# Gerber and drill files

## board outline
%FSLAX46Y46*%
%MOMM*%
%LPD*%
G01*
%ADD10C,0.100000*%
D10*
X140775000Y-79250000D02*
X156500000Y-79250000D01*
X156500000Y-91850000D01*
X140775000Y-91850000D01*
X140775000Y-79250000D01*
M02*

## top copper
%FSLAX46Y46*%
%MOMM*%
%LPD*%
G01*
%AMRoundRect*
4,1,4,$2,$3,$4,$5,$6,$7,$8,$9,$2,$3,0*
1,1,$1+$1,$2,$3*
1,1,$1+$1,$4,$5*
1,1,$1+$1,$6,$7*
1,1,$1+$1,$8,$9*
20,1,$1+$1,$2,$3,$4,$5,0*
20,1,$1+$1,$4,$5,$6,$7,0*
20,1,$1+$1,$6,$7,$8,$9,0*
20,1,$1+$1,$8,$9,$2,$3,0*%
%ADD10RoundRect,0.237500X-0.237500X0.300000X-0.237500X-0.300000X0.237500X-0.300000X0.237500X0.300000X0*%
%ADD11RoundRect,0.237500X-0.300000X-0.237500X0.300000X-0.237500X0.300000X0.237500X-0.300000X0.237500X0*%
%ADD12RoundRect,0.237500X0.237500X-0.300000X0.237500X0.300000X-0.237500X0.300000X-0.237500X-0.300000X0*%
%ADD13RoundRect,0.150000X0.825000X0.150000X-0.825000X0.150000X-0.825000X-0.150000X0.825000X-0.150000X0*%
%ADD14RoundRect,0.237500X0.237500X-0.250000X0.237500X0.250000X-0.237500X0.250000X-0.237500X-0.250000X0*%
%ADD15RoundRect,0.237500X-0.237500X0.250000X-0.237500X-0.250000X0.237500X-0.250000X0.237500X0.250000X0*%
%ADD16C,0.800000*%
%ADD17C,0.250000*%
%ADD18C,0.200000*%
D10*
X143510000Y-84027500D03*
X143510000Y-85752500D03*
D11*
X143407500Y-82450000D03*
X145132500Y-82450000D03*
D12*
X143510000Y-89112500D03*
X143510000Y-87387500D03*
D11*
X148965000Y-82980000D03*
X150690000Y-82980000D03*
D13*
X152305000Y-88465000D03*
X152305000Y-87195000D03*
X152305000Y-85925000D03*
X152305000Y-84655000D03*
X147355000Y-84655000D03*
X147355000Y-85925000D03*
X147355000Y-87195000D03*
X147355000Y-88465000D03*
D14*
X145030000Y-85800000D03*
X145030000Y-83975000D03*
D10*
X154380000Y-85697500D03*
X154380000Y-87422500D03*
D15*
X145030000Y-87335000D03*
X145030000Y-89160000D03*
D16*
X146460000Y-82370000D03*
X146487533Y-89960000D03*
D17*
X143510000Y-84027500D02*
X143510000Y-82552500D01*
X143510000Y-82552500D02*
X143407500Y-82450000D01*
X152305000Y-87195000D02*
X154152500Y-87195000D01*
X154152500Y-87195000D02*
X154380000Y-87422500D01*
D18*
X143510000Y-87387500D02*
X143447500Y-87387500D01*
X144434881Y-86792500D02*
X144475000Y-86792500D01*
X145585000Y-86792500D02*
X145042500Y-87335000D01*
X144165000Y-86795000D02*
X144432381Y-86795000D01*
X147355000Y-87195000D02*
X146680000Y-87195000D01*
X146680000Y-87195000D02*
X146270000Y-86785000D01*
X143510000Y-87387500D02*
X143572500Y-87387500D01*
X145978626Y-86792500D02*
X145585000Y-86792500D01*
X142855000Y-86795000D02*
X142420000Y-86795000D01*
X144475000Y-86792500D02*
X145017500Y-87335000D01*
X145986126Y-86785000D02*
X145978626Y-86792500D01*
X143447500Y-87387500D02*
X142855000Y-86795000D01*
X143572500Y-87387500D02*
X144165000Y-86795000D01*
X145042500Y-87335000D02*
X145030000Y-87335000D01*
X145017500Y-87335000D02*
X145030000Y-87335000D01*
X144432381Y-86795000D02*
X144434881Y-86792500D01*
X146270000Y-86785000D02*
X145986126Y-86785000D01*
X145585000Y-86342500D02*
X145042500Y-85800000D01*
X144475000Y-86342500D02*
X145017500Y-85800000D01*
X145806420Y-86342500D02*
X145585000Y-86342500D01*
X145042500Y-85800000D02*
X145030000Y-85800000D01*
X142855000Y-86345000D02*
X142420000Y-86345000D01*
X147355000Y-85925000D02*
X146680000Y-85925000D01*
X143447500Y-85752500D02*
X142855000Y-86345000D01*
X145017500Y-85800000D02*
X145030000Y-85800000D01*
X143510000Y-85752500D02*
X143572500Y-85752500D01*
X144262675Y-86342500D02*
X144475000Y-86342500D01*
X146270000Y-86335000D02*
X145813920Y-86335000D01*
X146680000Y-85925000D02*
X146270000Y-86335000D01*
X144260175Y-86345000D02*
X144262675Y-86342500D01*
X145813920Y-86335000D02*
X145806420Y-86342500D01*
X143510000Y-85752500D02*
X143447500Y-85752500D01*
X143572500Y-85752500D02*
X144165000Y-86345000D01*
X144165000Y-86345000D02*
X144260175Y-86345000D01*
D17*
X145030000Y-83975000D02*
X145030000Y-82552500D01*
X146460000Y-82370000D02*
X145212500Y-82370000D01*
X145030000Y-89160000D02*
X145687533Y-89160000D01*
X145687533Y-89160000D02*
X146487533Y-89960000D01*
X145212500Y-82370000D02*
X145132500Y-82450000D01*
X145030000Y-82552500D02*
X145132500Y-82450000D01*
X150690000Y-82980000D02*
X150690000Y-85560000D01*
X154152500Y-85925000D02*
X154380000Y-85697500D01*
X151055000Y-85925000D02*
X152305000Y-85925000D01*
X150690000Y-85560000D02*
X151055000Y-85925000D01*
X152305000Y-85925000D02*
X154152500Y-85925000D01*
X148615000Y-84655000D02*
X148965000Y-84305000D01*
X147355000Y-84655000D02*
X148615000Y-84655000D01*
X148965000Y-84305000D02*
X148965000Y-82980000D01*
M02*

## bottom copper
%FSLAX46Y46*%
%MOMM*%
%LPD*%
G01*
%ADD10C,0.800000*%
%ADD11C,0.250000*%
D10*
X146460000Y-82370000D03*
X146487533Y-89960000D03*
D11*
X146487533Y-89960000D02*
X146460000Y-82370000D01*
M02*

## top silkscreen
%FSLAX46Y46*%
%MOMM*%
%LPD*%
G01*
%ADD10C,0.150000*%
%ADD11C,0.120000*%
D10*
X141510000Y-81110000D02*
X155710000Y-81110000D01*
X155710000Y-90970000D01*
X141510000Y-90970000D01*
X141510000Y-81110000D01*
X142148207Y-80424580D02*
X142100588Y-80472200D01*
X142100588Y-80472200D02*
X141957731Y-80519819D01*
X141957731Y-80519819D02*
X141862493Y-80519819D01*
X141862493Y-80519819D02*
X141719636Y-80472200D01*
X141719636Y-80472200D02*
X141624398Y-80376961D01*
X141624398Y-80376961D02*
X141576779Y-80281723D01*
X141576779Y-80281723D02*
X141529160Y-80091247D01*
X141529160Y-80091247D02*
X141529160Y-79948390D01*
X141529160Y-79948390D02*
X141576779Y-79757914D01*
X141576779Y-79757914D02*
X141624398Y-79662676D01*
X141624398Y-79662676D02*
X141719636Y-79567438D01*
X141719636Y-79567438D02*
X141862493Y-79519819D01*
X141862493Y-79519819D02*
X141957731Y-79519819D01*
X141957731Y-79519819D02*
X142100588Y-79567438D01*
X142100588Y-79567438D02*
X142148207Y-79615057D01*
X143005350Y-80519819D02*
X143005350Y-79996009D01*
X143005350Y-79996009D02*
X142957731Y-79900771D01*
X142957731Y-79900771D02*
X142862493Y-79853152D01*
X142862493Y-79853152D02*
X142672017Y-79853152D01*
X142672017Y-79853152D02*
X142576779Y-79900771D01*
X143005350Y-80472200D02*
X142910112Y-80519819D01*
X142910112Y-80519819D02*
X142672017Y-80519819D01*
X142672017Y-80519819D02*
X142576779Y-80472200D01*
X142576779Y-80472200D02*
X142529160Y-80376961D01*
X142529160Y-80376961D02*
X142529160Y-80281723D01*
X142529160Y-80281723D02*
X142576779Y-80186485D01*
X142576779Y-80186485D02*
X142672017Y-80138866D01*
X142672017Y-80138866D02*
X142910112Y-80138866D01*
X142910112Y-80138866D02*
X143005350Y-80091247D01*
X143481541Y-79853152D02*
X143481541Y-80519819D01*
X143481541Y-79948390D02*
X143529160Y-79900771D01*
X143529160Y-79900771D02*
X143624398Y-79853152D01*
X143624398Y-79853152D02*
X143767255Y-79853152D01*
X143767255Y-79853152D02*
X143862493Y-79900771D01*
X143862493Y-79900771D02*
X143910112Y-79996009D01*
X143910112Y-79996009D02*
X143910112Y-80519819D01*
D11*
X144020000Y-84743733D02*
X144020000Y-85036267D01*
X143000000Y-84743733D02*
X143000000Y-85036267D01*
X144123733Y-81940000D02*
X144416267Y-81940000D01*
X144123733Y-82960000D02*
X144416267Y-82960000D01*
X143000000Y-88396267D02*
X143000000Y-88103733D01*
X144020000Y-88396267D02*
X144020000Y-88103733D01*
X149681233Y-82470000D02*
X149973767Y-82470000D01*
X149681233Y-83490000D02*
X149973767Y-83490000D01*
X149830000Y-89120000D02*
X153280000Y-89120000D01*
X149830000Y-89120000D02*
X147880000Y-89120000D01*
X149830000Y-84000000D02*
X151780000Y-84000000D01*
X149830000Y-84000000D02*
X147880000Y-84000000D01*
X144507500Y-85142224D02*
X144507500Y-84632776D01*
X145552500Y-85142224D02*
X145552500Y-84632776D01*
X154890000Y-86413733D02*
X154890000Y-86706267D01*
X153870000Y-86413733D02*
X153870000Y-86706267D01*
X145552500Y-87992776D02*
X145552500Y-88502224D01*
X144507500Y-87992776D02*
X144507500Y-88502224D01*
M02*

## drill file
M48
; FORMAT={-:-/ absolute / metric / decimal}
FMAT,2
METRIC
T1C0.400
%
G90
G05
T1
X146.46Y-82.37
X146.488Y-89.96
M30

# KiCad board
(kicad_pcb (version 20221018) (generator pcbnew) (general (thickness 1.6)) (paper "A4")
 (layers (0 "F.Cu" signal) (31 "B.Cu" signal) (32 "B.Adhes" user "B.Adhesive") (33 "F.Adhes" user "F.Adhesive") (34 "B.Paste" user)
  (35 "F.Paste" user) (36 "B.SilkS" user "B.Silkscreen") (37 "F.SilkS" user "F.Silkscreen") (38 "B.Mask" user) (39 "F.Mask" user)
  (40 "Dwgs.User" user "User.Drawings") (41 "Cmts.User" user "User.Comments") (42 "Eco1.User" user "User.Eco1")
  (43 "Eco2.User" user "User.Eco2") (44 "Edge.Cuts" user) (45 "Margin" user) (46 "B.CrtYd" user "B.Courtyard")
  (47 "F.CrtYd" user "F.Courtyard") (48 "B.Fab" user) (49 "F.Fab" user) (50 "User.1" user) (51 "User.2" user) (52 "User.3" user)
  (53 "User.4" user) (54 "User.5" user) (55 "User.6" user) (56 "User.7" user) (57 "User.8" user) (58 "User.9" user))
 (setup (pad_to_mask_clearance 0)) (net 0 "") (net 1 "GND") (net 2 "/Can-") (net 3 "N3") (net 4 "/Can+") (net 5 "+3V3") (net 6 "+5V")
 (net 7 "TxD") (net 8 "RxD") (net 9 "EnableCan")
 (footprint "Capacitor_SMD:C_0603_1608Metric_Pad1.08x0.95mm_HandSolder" (layer "F.Cu") (at 143.51 84.89 -90)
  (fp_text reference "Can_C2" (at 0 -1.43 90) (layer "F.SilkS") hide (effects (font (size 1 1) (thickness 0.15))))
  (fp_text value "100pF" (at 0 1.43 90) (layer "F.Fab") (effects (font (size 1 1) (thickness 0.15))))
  (fp_line (start -0.146267 -0.51) (end 0.146267 -0.51) (stroke (width 0.12) (type solid)) (layer "F.SilkS"))
  (fp_line (start -0.146267 0.51) (end 0.146267 0.51) (stroke (width 0.12) (type solid)) (layer "F.SilkS"))
  (pad "1" smd roundrect (at -0.8625 0 270) (size 1.075 0.95) (layers "F.Cu" "F.Paste" "F.Mask") (roundrect_rratio 0.25) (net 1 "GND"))
  (pad "2" smd roundrect (at 0.8625 0 270) (size 1.075 0.95) (layers "F.Cu" "F.Paste" "F.Mask") (roundrect_rratio 0.25) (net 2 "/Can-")))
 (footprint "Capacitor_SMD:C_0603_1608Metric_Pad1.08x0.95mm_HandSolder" (layer "F.Cu") (at 144.27 82.45)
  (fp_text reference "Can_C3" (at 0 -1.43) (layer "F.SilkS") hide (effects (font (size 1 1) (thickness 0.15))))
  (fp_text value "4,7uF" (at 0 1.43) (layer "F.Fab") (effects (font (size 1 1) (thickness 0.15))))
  (fp_line (start -0.146267 -0.51) (end 0.146267 -0.51) (stroke (width 0.12) (type solid)) (layer "F.SilkS"))
  (fp_line (start -0.146267 0.51) (end 0.146267 0.51) (stroke (width 0.12) (type solid)) (layer "F.SilkS"))
  (pad "1" smd roundrect (at -0.8625 0) (size 1.075 0.95) (layers "F.Cu" "F.Paste" "F.Mask") (roundrect_rratio 0.25) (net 1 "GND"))
  (pad "2" smd roundrect (at 0.8625 0) (size 1.075 0.95) (layers "F.Cu" "F.Paste" "F.Mask") (roundrect_rratio 0.25) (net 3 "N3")))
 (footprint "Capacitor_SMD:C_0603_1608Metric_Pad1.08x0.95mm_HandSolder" (layer "F.Cu") (at 143.51 88.25 90)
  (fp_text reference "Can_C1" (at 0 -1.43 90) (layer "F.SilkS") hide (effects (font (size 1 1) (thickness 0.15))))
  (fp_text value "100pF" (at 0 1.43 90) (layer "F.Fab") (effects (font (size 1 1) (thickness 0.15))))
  (fp_line (start -0.146267 -0.51) (end 0.146267 -0.51) (stroke (width 0.12) (type solid)) (layer "F.SilkS"))
  (fp_line (start -0.146267 0.51) (end 0.146267 0.51) (stroke (width 0.12) (type solid)) (layer "F.SilkS"))
  (pad "1" smd roundrect (at -0.8625 0 90) (size 1.075 0.95) (layers "F.Cu" "F.Paste" "F.Mask") (roundrect_rratio 0.25) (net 1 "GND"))
  (pad "2" smd roundrect (at 0.8625 0 90) (size 1.075 0.95) (layers "F.Cu" "F.Paste" "F.Mask") (roundrect_rratio 0.25) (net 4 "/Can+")))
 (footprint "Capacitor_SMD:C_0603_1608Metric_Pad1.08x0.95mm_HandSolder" (layer "F.Cu") (at 149.8275 82.98)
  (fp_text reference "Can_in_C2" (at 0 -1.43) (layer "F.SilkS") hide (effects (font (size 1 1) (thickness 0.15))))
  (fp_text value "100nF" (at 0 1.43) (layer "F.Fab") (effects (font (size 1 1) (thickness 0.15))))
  (fp_line (start -0.146267 -0.51) (end 0.146267 -0.51) (stroke (width 0.12) (type solid)) (layer "F.SilkS"))
  (fp_line (start -0.146267 0.51) (end 0.146267 0.51) (stroke (width 0.12) (type solid)) (layer "F.SilkS"))
  (pad "1" smd roundrect (at -0.8625 0) (size 1.075 0.95) (layers "F.Cu" "F.Paste" "F.Mask") (roundrect_rratio 0.25) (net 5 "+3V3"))
  (pad "2" smd roundrect (at 0.8625 0) (size 1.075 0.95) (layers "F.Cu" "F.Paste" "F.Mask") (roundrect_rratio 0.25) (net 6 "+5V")))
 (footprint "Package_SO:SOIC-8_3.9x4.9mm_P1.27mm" (layer "F.Cu") (at 149.83 86.56 180)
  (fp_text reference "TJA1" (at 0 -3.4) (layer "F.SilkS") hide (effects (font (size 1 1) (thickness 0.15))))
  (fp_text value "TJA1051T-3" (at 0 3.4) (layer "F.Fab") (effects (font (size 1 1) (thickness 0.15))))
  (fp_line (start 0 -2.56) (end -3.45 -2.56) (stroke (width 0.12) (type solid)) (layer "F.SilkS"))
  (fp_line (start 0 -2.56) (end 1.95 -2.56) (stroke (width 0.12) (type solid)) (layer "F.SilkS"))
  (fp_line (start 0 2.56) (end -1.95 2.56) (stroke (width 0.12) (type solid)) (layer "F.SilkS"))
  (fp_line (start 0 2.56) (end 1.95 2.56) (stroke (width 0.12) (type solid)) (layer "F.SilkS"))
  (pad "1" smd roundrect (at -2.475 -1.905 180) (size 1.95 0.6) (layers "F.Cu" "F.Paste" "F.Mask") (roundrect_rratio 0.25) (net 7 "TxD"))
  (pad "2" smd roundrect (at -2.475 -0.635 180) (size 1.95 0.6) (layers "F.Cu" "F.Paste" "F.Mask") (roundrect_rratio 0.25) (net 1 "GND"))
  (pad "3" smd roundrect (at -2.475 0.635 180) (size 1.95 0.6) (layers "F.Cu" "F.Paste" "F.Mask") (roundrect_rratio 0.25) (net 6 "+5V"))
  (pad "4" smd roundrect (at -2.475 1.905 180) (size 1.95 0.6) (layers "F.Cu" "F.Paste" "F.Mask") (roundrect_rratio 0.25) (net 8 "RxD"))
  (pad "5" smd roundrect (at 2.475 1.905 180) (size 1.95 0.6) (layers "F.Cu" "F.Paste" "F.Mask") (roundrect_rratio 0.25) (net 5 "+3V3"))
  (pad "6" smd roundrect (at 2.475 0.635 180) (size 1.95 0.6) (layers "F.Cu" "F.Paste" "F.Mask") (roundrect_rratio 0.25) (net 2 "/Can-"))
  (pad "7" smd roundrect (at 2.475 -0.635 180) (size 1.95 0.6) (layers "F.Cu" "F.Paste" "F.Mask") (roundrect_rratio 0.25) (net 4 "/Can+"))
  (pad "8" smd roundrect (at 2.475 -1.905 180) (size 1.95 0.6) (layers "F.Cu" "F.Paste" "F.Mask") (roundrect_rratio 0.25)
   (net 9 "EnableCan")))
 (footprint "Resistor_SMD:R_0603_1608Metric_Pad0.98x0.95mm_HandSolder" (layer "F.Cu") (at 145.03 84.8875 90)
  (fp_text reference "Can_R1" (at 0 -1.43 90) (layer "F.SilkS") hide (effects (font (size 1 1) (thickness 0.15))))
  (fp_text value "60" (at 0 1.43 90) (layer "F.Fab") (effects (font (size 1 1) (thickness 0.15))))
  (fp_line (start -0.254724 -0.5225) (end 0.254724 -0.5225) (stroke (width 0.12) (type solid)) (layer "F.SilkS"))
  (fp_line (start -0.254724 0.5225) (end 0.254724 0.5225) (stroke (width 0.12) (type solid)) (layer "F.SilkS"))
  (pad "1" smd roundrect (at -0.9125 0 90) (size 0.975 0.95) (layers "F.Cu" "F.Paste" "F.Mask") (roundrect_rratio 0.25) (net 2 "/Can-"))
  (pad "2" smd roundrect (at 0.9125 0 90) (size 0.975 0.95) (layers "F.Cu" "F.Paste" "F.Mask") (roundrect_rratio 0.25) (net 3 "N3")))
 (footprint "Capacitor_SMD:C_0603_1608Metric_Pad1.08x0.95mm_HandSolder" (layer "F.Cu") (at 154.38 86.56 -90)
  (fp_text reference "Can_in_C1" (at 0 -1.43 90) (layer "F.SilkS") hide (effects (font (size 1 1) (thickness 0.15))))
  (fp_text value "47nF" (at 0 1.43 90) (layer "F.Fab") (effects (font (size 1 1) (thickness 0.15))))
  (fp_line (start -0.146267 -0.51) (end 0.146267 -0.51) (stroke (width 0.12) (type solid)) (layer "F.SilkS"))
  (fp_line (start -0.146267 0.51) (end 0.146267 0.51) (stroke (width 0.12) (type solid)) (layer "F.SilkS"))
  (pad "1" smd roundrect (at -0.8625 0 270) (size 1.075 0.95) (layers "F.Cu" "F.Paste" "F.Mask") (roundrect_rratio 0.25) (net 6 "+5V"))
  (pad "2" smd roundrect (at 0.8625 0 270) (size 1.075 0.95) (layers "F.Cu" "F.Paste" "F.Mask") (roundrect_rratio 0.25) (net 1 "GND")))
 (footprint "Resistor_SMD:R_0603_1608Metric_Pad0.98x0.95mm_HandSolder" (layer "F.Cu") (at 145.03 88.2475 -90)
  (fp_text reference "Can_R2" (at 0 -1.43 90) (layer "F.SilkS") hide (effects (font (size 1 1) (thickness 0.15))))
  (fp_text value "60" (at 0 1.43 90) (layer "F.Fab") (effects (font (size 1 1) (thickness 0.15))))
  (fp_line (start -0.254724 -0.5225) (end 0.254724 -0.5225) (stroke (width 0.12) (type solid)) (layer "F.SilkS"))
  (fp_line (start -0.254724 0.5225) (end 0.254724 0.5225) (stroke (width 0.12) (type solid)) (layer "F.SilkS"))
  (pad "1" smd roundrect (at -0.9125 0 270) (size 0.975 0.95) (layers "F.Cu" "F.Paste" "F.Mask") (roundrect_rratio 0.25) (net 4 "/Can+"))
  (pad "2" smd roundrect (at 0.9125 0 270) (size 0.975 0.95) (layers "F.Cu" "F.Paste" "F.Mask") (roundrect_rratio 0.25) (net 3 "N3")))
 (gr_rect (start 141.51 81.11) (end 155.71 90.97) (stroke (width 0.15) (type default)) (fill none) (layer "F.SilkS"))
 (gr_rect (start 140.775 79.25) (end 156.5 91.85) (stroke (width 0.1) (type default)) (fill none) (layer "Edge.Cuts"))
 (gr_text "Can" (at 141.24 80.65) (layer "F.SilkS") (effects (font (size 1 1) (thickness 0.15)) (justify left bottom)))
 (segment (start 143.51 84.0275) (end 143.51 82.5525) (width 0.25) (layer "F.Cu") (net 1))
 (segment (start 143.51 82.5525) (end 143.4075 82.45) (width 0.25) (layer "F.Cu") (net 1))
 (segment (start 152.305 87.195) (end 154.1525 87.195) (width 0.25) (layer "F.Cu") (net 1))
 (segment (start 154.1525 87.195) (end 154.38 87.4225) (width 0.25) (layer "F.Cu") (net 1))
 (segment (start 143.51 87.3875) (end 143.4475 87.3875) (width 0.2) (layer "F.Cu") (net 4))
 (segment (start 144.434881 86.7925) (end 144.475 86.7925) (width 0.2) (layer "F.Cu") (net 4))
 (segment (start 145.585 86.7925) (end 145.0425 87.335) (width 0.2) (layer "F.Cu") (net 4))
 (segment (start 144.165 86.795) (end 144.432381 86.795) (width 0.2) (layer "F.Cu") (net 4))
 (segment (start 147.355 87.195) (end 146.68 87.195) (width 0.2) (layer "F.Cu") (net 4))
 (segment (start 146.68 87.195) (end 146.27 86.785) (width 0.2) (layer "F.Cu") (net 4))
 (segment (start 143.51 87.3875) (end 143.5725 87.3875) (width 0.2) (layer "F.Cu") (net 4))
 (segment (start 145.978626 86.7925) (end 145.585 86.7925) (width 0.2) (layer "F.Cu") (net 4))
 (segment (start 142.855 86.795) (end 142.42 86.795) (width 0.2) (layer "F.Cu") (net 4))
 (segment (start 144.475 86.7925) (end 145.0175 87.335) (width 0.2) (layer "F.Cu") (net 4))
 (segment (start 145.986126 86.785) (end 145.978626 86.7925) (width 0.2) (layer "F.Cu") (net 4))
 (segment (start 143.4475 87.3875) (end 142.855 86.795) (width 0.2) (layer "F.Cu") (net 4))
 (segment (start 143.5725 87.3875) (end 144.165 86.795) (width 0.2) (layer "F.Cu") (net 4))
 (segment (start 145.0425 87.335) (end 145.03 87.335) (width 0.2) (layer "F.Cu") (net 4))
 (segment (start 145.0175 87.335) (end 145.03 87.335) (width 0.2) (layer "F.Cu") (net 4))
 (segment (start 144.432381 86.795) (end 144.434881 86.7925) (width 0.2) (layer "F.Cu") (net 4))
 (segment (start 146.27 86.785) (end 145.986126 86.785) (width 0.2) (layer "F.Cu") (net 4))
 (segment (start 145.585 86.3425) (end 145.0425 85.8) (width 0.2) (layer "F.Cu") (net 2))
 (segment (start 144.475 86.3425) (end 145.0175 85.8) (width 0.2) (layer "F.Cu") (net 2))
 (segment (start 145.80642 86.3425) (end 145.585 86.3425) (width 0.2) (layer "F.Cu") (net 2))
 (segment (start 145.0425 85.8) (end 145.03 85.8) (width 0.2) (layer "F.Cu") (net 2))
 (segment (start 142.855 86.345) (end 142.42 86.345) (width 0.2) (layer "F.Cu") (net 2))
 (segment (start 147.355 85.925) (end 146.68 85.925) (width 0.2) (layer "F.Cu") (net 2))
 (segment (start 143.4475 85.7525) (end 142.855 86.345) (width 0.2) (layer "F.Cu") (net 2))
 (segment (start 145.0175 85.8) (end 145.03 85.8) (width 0.2) (layer "F.Cu") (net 2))
 (segment (start 143.51 85.7525) (end 143.5725 85.7525) (width 0.2) (layer "F.Cu") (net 2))
 (segment (start 144.262675 86.3425) (end 144.475 86.3425) (width 0.2) (layer "F.Cu") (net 2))
 (segment (start 146.27 86.335) (end 145.81392 86.335) (width 0.2) (layer "F.Cu") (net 2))
 (segment (start 146.68 85.925) (end 146.27 86.335) (width 0.2) (layer "F.Cu") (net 2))
 (segment (start 144.260175 86.345) (end 144.262675 86.3425) (width 0.2) (layer "F.Cu") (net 2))
 (segment (start 145.81392 86.335) (end 145.80642 86.3425) (width 0.2) (layer "F.Cu") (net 2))
 (segment (start 143.51 85.7525) (end 143.4475 85.7525) (width 0.2) (layer "F.Cu") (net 2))
 (segment (start 143.5725 85.7525) (end 144.165 86.345) (width 0.2) (layer "F.Cu") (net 2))
 (segment (start 144.165 86.345) (end 144.260175 86.345) (width 0.2) (layer "F.Cu") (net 2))
 (segment (start 145.03 83.975) (end 145.03 82.5525) (width 0.25) (layer "F.Cu") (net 3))
 (segment (start 146.46 82.37) (end 145.2125 82.37) (width 0.25) (layer "F.Cu") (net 3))
 (segment (start 145.03 89.16) (end 145.687533 89.16) (width 0.25) (layer "F.Cu") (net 3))
 (segment (start 145.687533 89.16) (end 146.487533 89.96) (width 0.25) (layer "F.Cu") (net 3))
 (segment (start 145.2125 82.37) (end 145.1325 82.45) (width 0.25) (layer "F.Cu") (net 3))
 (segment (start 145.03 82.5525) (end 145.1325 82.45) (width 0.25) (layer "F.Cu") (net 3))
 (via (at 146.46 82.37) (size 0.8) (drill 0.4) (layers "F.Cu" "B.Cu") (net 3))
 (via (at 146.487533 89.96) (size 0.8) (drill 0.4) (layers "F.Cu" "B.Cu") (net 3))
 (segment (start 146.487533 89.96) (end 146.46 82.37) (width 0.25) (layer "B.Cu") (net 3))
 (segment (start 150.69 82.98) (end 150.69 85.56) (width 0.25) (layer "F.Cu") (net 6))
 (segment (start 154.1525 85.925) (end 154.38 85.6975) (width 0.25) (layer "F.Cu") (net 6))
 (segment (start 151.055 85.925) (end 152.305 85.925) (width 0.25) (layer "F.Cu") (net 6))
 (segment (start 150.69 85.56) (end 151.055 85.925) (width 0.25) (layer "F.Cu") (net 6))
 (segment (start 152.305 85.925) (end 154.1525 85.925) (width 0.25) (layer "F.Cu") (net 6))
 (segment (start 148.615 84.655) (end 148.965 84.305) (width 0.25) (layer "F.Cu") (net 5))
 (segment (start 147.355 84.655) (end 148.615 84.655) (width 0.25) (layer "F.Cu") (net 5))
 (segment (start 148.965 84.305) (end 148.965 82.98) (width 0.25) (layer "F.Cu") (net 5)))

